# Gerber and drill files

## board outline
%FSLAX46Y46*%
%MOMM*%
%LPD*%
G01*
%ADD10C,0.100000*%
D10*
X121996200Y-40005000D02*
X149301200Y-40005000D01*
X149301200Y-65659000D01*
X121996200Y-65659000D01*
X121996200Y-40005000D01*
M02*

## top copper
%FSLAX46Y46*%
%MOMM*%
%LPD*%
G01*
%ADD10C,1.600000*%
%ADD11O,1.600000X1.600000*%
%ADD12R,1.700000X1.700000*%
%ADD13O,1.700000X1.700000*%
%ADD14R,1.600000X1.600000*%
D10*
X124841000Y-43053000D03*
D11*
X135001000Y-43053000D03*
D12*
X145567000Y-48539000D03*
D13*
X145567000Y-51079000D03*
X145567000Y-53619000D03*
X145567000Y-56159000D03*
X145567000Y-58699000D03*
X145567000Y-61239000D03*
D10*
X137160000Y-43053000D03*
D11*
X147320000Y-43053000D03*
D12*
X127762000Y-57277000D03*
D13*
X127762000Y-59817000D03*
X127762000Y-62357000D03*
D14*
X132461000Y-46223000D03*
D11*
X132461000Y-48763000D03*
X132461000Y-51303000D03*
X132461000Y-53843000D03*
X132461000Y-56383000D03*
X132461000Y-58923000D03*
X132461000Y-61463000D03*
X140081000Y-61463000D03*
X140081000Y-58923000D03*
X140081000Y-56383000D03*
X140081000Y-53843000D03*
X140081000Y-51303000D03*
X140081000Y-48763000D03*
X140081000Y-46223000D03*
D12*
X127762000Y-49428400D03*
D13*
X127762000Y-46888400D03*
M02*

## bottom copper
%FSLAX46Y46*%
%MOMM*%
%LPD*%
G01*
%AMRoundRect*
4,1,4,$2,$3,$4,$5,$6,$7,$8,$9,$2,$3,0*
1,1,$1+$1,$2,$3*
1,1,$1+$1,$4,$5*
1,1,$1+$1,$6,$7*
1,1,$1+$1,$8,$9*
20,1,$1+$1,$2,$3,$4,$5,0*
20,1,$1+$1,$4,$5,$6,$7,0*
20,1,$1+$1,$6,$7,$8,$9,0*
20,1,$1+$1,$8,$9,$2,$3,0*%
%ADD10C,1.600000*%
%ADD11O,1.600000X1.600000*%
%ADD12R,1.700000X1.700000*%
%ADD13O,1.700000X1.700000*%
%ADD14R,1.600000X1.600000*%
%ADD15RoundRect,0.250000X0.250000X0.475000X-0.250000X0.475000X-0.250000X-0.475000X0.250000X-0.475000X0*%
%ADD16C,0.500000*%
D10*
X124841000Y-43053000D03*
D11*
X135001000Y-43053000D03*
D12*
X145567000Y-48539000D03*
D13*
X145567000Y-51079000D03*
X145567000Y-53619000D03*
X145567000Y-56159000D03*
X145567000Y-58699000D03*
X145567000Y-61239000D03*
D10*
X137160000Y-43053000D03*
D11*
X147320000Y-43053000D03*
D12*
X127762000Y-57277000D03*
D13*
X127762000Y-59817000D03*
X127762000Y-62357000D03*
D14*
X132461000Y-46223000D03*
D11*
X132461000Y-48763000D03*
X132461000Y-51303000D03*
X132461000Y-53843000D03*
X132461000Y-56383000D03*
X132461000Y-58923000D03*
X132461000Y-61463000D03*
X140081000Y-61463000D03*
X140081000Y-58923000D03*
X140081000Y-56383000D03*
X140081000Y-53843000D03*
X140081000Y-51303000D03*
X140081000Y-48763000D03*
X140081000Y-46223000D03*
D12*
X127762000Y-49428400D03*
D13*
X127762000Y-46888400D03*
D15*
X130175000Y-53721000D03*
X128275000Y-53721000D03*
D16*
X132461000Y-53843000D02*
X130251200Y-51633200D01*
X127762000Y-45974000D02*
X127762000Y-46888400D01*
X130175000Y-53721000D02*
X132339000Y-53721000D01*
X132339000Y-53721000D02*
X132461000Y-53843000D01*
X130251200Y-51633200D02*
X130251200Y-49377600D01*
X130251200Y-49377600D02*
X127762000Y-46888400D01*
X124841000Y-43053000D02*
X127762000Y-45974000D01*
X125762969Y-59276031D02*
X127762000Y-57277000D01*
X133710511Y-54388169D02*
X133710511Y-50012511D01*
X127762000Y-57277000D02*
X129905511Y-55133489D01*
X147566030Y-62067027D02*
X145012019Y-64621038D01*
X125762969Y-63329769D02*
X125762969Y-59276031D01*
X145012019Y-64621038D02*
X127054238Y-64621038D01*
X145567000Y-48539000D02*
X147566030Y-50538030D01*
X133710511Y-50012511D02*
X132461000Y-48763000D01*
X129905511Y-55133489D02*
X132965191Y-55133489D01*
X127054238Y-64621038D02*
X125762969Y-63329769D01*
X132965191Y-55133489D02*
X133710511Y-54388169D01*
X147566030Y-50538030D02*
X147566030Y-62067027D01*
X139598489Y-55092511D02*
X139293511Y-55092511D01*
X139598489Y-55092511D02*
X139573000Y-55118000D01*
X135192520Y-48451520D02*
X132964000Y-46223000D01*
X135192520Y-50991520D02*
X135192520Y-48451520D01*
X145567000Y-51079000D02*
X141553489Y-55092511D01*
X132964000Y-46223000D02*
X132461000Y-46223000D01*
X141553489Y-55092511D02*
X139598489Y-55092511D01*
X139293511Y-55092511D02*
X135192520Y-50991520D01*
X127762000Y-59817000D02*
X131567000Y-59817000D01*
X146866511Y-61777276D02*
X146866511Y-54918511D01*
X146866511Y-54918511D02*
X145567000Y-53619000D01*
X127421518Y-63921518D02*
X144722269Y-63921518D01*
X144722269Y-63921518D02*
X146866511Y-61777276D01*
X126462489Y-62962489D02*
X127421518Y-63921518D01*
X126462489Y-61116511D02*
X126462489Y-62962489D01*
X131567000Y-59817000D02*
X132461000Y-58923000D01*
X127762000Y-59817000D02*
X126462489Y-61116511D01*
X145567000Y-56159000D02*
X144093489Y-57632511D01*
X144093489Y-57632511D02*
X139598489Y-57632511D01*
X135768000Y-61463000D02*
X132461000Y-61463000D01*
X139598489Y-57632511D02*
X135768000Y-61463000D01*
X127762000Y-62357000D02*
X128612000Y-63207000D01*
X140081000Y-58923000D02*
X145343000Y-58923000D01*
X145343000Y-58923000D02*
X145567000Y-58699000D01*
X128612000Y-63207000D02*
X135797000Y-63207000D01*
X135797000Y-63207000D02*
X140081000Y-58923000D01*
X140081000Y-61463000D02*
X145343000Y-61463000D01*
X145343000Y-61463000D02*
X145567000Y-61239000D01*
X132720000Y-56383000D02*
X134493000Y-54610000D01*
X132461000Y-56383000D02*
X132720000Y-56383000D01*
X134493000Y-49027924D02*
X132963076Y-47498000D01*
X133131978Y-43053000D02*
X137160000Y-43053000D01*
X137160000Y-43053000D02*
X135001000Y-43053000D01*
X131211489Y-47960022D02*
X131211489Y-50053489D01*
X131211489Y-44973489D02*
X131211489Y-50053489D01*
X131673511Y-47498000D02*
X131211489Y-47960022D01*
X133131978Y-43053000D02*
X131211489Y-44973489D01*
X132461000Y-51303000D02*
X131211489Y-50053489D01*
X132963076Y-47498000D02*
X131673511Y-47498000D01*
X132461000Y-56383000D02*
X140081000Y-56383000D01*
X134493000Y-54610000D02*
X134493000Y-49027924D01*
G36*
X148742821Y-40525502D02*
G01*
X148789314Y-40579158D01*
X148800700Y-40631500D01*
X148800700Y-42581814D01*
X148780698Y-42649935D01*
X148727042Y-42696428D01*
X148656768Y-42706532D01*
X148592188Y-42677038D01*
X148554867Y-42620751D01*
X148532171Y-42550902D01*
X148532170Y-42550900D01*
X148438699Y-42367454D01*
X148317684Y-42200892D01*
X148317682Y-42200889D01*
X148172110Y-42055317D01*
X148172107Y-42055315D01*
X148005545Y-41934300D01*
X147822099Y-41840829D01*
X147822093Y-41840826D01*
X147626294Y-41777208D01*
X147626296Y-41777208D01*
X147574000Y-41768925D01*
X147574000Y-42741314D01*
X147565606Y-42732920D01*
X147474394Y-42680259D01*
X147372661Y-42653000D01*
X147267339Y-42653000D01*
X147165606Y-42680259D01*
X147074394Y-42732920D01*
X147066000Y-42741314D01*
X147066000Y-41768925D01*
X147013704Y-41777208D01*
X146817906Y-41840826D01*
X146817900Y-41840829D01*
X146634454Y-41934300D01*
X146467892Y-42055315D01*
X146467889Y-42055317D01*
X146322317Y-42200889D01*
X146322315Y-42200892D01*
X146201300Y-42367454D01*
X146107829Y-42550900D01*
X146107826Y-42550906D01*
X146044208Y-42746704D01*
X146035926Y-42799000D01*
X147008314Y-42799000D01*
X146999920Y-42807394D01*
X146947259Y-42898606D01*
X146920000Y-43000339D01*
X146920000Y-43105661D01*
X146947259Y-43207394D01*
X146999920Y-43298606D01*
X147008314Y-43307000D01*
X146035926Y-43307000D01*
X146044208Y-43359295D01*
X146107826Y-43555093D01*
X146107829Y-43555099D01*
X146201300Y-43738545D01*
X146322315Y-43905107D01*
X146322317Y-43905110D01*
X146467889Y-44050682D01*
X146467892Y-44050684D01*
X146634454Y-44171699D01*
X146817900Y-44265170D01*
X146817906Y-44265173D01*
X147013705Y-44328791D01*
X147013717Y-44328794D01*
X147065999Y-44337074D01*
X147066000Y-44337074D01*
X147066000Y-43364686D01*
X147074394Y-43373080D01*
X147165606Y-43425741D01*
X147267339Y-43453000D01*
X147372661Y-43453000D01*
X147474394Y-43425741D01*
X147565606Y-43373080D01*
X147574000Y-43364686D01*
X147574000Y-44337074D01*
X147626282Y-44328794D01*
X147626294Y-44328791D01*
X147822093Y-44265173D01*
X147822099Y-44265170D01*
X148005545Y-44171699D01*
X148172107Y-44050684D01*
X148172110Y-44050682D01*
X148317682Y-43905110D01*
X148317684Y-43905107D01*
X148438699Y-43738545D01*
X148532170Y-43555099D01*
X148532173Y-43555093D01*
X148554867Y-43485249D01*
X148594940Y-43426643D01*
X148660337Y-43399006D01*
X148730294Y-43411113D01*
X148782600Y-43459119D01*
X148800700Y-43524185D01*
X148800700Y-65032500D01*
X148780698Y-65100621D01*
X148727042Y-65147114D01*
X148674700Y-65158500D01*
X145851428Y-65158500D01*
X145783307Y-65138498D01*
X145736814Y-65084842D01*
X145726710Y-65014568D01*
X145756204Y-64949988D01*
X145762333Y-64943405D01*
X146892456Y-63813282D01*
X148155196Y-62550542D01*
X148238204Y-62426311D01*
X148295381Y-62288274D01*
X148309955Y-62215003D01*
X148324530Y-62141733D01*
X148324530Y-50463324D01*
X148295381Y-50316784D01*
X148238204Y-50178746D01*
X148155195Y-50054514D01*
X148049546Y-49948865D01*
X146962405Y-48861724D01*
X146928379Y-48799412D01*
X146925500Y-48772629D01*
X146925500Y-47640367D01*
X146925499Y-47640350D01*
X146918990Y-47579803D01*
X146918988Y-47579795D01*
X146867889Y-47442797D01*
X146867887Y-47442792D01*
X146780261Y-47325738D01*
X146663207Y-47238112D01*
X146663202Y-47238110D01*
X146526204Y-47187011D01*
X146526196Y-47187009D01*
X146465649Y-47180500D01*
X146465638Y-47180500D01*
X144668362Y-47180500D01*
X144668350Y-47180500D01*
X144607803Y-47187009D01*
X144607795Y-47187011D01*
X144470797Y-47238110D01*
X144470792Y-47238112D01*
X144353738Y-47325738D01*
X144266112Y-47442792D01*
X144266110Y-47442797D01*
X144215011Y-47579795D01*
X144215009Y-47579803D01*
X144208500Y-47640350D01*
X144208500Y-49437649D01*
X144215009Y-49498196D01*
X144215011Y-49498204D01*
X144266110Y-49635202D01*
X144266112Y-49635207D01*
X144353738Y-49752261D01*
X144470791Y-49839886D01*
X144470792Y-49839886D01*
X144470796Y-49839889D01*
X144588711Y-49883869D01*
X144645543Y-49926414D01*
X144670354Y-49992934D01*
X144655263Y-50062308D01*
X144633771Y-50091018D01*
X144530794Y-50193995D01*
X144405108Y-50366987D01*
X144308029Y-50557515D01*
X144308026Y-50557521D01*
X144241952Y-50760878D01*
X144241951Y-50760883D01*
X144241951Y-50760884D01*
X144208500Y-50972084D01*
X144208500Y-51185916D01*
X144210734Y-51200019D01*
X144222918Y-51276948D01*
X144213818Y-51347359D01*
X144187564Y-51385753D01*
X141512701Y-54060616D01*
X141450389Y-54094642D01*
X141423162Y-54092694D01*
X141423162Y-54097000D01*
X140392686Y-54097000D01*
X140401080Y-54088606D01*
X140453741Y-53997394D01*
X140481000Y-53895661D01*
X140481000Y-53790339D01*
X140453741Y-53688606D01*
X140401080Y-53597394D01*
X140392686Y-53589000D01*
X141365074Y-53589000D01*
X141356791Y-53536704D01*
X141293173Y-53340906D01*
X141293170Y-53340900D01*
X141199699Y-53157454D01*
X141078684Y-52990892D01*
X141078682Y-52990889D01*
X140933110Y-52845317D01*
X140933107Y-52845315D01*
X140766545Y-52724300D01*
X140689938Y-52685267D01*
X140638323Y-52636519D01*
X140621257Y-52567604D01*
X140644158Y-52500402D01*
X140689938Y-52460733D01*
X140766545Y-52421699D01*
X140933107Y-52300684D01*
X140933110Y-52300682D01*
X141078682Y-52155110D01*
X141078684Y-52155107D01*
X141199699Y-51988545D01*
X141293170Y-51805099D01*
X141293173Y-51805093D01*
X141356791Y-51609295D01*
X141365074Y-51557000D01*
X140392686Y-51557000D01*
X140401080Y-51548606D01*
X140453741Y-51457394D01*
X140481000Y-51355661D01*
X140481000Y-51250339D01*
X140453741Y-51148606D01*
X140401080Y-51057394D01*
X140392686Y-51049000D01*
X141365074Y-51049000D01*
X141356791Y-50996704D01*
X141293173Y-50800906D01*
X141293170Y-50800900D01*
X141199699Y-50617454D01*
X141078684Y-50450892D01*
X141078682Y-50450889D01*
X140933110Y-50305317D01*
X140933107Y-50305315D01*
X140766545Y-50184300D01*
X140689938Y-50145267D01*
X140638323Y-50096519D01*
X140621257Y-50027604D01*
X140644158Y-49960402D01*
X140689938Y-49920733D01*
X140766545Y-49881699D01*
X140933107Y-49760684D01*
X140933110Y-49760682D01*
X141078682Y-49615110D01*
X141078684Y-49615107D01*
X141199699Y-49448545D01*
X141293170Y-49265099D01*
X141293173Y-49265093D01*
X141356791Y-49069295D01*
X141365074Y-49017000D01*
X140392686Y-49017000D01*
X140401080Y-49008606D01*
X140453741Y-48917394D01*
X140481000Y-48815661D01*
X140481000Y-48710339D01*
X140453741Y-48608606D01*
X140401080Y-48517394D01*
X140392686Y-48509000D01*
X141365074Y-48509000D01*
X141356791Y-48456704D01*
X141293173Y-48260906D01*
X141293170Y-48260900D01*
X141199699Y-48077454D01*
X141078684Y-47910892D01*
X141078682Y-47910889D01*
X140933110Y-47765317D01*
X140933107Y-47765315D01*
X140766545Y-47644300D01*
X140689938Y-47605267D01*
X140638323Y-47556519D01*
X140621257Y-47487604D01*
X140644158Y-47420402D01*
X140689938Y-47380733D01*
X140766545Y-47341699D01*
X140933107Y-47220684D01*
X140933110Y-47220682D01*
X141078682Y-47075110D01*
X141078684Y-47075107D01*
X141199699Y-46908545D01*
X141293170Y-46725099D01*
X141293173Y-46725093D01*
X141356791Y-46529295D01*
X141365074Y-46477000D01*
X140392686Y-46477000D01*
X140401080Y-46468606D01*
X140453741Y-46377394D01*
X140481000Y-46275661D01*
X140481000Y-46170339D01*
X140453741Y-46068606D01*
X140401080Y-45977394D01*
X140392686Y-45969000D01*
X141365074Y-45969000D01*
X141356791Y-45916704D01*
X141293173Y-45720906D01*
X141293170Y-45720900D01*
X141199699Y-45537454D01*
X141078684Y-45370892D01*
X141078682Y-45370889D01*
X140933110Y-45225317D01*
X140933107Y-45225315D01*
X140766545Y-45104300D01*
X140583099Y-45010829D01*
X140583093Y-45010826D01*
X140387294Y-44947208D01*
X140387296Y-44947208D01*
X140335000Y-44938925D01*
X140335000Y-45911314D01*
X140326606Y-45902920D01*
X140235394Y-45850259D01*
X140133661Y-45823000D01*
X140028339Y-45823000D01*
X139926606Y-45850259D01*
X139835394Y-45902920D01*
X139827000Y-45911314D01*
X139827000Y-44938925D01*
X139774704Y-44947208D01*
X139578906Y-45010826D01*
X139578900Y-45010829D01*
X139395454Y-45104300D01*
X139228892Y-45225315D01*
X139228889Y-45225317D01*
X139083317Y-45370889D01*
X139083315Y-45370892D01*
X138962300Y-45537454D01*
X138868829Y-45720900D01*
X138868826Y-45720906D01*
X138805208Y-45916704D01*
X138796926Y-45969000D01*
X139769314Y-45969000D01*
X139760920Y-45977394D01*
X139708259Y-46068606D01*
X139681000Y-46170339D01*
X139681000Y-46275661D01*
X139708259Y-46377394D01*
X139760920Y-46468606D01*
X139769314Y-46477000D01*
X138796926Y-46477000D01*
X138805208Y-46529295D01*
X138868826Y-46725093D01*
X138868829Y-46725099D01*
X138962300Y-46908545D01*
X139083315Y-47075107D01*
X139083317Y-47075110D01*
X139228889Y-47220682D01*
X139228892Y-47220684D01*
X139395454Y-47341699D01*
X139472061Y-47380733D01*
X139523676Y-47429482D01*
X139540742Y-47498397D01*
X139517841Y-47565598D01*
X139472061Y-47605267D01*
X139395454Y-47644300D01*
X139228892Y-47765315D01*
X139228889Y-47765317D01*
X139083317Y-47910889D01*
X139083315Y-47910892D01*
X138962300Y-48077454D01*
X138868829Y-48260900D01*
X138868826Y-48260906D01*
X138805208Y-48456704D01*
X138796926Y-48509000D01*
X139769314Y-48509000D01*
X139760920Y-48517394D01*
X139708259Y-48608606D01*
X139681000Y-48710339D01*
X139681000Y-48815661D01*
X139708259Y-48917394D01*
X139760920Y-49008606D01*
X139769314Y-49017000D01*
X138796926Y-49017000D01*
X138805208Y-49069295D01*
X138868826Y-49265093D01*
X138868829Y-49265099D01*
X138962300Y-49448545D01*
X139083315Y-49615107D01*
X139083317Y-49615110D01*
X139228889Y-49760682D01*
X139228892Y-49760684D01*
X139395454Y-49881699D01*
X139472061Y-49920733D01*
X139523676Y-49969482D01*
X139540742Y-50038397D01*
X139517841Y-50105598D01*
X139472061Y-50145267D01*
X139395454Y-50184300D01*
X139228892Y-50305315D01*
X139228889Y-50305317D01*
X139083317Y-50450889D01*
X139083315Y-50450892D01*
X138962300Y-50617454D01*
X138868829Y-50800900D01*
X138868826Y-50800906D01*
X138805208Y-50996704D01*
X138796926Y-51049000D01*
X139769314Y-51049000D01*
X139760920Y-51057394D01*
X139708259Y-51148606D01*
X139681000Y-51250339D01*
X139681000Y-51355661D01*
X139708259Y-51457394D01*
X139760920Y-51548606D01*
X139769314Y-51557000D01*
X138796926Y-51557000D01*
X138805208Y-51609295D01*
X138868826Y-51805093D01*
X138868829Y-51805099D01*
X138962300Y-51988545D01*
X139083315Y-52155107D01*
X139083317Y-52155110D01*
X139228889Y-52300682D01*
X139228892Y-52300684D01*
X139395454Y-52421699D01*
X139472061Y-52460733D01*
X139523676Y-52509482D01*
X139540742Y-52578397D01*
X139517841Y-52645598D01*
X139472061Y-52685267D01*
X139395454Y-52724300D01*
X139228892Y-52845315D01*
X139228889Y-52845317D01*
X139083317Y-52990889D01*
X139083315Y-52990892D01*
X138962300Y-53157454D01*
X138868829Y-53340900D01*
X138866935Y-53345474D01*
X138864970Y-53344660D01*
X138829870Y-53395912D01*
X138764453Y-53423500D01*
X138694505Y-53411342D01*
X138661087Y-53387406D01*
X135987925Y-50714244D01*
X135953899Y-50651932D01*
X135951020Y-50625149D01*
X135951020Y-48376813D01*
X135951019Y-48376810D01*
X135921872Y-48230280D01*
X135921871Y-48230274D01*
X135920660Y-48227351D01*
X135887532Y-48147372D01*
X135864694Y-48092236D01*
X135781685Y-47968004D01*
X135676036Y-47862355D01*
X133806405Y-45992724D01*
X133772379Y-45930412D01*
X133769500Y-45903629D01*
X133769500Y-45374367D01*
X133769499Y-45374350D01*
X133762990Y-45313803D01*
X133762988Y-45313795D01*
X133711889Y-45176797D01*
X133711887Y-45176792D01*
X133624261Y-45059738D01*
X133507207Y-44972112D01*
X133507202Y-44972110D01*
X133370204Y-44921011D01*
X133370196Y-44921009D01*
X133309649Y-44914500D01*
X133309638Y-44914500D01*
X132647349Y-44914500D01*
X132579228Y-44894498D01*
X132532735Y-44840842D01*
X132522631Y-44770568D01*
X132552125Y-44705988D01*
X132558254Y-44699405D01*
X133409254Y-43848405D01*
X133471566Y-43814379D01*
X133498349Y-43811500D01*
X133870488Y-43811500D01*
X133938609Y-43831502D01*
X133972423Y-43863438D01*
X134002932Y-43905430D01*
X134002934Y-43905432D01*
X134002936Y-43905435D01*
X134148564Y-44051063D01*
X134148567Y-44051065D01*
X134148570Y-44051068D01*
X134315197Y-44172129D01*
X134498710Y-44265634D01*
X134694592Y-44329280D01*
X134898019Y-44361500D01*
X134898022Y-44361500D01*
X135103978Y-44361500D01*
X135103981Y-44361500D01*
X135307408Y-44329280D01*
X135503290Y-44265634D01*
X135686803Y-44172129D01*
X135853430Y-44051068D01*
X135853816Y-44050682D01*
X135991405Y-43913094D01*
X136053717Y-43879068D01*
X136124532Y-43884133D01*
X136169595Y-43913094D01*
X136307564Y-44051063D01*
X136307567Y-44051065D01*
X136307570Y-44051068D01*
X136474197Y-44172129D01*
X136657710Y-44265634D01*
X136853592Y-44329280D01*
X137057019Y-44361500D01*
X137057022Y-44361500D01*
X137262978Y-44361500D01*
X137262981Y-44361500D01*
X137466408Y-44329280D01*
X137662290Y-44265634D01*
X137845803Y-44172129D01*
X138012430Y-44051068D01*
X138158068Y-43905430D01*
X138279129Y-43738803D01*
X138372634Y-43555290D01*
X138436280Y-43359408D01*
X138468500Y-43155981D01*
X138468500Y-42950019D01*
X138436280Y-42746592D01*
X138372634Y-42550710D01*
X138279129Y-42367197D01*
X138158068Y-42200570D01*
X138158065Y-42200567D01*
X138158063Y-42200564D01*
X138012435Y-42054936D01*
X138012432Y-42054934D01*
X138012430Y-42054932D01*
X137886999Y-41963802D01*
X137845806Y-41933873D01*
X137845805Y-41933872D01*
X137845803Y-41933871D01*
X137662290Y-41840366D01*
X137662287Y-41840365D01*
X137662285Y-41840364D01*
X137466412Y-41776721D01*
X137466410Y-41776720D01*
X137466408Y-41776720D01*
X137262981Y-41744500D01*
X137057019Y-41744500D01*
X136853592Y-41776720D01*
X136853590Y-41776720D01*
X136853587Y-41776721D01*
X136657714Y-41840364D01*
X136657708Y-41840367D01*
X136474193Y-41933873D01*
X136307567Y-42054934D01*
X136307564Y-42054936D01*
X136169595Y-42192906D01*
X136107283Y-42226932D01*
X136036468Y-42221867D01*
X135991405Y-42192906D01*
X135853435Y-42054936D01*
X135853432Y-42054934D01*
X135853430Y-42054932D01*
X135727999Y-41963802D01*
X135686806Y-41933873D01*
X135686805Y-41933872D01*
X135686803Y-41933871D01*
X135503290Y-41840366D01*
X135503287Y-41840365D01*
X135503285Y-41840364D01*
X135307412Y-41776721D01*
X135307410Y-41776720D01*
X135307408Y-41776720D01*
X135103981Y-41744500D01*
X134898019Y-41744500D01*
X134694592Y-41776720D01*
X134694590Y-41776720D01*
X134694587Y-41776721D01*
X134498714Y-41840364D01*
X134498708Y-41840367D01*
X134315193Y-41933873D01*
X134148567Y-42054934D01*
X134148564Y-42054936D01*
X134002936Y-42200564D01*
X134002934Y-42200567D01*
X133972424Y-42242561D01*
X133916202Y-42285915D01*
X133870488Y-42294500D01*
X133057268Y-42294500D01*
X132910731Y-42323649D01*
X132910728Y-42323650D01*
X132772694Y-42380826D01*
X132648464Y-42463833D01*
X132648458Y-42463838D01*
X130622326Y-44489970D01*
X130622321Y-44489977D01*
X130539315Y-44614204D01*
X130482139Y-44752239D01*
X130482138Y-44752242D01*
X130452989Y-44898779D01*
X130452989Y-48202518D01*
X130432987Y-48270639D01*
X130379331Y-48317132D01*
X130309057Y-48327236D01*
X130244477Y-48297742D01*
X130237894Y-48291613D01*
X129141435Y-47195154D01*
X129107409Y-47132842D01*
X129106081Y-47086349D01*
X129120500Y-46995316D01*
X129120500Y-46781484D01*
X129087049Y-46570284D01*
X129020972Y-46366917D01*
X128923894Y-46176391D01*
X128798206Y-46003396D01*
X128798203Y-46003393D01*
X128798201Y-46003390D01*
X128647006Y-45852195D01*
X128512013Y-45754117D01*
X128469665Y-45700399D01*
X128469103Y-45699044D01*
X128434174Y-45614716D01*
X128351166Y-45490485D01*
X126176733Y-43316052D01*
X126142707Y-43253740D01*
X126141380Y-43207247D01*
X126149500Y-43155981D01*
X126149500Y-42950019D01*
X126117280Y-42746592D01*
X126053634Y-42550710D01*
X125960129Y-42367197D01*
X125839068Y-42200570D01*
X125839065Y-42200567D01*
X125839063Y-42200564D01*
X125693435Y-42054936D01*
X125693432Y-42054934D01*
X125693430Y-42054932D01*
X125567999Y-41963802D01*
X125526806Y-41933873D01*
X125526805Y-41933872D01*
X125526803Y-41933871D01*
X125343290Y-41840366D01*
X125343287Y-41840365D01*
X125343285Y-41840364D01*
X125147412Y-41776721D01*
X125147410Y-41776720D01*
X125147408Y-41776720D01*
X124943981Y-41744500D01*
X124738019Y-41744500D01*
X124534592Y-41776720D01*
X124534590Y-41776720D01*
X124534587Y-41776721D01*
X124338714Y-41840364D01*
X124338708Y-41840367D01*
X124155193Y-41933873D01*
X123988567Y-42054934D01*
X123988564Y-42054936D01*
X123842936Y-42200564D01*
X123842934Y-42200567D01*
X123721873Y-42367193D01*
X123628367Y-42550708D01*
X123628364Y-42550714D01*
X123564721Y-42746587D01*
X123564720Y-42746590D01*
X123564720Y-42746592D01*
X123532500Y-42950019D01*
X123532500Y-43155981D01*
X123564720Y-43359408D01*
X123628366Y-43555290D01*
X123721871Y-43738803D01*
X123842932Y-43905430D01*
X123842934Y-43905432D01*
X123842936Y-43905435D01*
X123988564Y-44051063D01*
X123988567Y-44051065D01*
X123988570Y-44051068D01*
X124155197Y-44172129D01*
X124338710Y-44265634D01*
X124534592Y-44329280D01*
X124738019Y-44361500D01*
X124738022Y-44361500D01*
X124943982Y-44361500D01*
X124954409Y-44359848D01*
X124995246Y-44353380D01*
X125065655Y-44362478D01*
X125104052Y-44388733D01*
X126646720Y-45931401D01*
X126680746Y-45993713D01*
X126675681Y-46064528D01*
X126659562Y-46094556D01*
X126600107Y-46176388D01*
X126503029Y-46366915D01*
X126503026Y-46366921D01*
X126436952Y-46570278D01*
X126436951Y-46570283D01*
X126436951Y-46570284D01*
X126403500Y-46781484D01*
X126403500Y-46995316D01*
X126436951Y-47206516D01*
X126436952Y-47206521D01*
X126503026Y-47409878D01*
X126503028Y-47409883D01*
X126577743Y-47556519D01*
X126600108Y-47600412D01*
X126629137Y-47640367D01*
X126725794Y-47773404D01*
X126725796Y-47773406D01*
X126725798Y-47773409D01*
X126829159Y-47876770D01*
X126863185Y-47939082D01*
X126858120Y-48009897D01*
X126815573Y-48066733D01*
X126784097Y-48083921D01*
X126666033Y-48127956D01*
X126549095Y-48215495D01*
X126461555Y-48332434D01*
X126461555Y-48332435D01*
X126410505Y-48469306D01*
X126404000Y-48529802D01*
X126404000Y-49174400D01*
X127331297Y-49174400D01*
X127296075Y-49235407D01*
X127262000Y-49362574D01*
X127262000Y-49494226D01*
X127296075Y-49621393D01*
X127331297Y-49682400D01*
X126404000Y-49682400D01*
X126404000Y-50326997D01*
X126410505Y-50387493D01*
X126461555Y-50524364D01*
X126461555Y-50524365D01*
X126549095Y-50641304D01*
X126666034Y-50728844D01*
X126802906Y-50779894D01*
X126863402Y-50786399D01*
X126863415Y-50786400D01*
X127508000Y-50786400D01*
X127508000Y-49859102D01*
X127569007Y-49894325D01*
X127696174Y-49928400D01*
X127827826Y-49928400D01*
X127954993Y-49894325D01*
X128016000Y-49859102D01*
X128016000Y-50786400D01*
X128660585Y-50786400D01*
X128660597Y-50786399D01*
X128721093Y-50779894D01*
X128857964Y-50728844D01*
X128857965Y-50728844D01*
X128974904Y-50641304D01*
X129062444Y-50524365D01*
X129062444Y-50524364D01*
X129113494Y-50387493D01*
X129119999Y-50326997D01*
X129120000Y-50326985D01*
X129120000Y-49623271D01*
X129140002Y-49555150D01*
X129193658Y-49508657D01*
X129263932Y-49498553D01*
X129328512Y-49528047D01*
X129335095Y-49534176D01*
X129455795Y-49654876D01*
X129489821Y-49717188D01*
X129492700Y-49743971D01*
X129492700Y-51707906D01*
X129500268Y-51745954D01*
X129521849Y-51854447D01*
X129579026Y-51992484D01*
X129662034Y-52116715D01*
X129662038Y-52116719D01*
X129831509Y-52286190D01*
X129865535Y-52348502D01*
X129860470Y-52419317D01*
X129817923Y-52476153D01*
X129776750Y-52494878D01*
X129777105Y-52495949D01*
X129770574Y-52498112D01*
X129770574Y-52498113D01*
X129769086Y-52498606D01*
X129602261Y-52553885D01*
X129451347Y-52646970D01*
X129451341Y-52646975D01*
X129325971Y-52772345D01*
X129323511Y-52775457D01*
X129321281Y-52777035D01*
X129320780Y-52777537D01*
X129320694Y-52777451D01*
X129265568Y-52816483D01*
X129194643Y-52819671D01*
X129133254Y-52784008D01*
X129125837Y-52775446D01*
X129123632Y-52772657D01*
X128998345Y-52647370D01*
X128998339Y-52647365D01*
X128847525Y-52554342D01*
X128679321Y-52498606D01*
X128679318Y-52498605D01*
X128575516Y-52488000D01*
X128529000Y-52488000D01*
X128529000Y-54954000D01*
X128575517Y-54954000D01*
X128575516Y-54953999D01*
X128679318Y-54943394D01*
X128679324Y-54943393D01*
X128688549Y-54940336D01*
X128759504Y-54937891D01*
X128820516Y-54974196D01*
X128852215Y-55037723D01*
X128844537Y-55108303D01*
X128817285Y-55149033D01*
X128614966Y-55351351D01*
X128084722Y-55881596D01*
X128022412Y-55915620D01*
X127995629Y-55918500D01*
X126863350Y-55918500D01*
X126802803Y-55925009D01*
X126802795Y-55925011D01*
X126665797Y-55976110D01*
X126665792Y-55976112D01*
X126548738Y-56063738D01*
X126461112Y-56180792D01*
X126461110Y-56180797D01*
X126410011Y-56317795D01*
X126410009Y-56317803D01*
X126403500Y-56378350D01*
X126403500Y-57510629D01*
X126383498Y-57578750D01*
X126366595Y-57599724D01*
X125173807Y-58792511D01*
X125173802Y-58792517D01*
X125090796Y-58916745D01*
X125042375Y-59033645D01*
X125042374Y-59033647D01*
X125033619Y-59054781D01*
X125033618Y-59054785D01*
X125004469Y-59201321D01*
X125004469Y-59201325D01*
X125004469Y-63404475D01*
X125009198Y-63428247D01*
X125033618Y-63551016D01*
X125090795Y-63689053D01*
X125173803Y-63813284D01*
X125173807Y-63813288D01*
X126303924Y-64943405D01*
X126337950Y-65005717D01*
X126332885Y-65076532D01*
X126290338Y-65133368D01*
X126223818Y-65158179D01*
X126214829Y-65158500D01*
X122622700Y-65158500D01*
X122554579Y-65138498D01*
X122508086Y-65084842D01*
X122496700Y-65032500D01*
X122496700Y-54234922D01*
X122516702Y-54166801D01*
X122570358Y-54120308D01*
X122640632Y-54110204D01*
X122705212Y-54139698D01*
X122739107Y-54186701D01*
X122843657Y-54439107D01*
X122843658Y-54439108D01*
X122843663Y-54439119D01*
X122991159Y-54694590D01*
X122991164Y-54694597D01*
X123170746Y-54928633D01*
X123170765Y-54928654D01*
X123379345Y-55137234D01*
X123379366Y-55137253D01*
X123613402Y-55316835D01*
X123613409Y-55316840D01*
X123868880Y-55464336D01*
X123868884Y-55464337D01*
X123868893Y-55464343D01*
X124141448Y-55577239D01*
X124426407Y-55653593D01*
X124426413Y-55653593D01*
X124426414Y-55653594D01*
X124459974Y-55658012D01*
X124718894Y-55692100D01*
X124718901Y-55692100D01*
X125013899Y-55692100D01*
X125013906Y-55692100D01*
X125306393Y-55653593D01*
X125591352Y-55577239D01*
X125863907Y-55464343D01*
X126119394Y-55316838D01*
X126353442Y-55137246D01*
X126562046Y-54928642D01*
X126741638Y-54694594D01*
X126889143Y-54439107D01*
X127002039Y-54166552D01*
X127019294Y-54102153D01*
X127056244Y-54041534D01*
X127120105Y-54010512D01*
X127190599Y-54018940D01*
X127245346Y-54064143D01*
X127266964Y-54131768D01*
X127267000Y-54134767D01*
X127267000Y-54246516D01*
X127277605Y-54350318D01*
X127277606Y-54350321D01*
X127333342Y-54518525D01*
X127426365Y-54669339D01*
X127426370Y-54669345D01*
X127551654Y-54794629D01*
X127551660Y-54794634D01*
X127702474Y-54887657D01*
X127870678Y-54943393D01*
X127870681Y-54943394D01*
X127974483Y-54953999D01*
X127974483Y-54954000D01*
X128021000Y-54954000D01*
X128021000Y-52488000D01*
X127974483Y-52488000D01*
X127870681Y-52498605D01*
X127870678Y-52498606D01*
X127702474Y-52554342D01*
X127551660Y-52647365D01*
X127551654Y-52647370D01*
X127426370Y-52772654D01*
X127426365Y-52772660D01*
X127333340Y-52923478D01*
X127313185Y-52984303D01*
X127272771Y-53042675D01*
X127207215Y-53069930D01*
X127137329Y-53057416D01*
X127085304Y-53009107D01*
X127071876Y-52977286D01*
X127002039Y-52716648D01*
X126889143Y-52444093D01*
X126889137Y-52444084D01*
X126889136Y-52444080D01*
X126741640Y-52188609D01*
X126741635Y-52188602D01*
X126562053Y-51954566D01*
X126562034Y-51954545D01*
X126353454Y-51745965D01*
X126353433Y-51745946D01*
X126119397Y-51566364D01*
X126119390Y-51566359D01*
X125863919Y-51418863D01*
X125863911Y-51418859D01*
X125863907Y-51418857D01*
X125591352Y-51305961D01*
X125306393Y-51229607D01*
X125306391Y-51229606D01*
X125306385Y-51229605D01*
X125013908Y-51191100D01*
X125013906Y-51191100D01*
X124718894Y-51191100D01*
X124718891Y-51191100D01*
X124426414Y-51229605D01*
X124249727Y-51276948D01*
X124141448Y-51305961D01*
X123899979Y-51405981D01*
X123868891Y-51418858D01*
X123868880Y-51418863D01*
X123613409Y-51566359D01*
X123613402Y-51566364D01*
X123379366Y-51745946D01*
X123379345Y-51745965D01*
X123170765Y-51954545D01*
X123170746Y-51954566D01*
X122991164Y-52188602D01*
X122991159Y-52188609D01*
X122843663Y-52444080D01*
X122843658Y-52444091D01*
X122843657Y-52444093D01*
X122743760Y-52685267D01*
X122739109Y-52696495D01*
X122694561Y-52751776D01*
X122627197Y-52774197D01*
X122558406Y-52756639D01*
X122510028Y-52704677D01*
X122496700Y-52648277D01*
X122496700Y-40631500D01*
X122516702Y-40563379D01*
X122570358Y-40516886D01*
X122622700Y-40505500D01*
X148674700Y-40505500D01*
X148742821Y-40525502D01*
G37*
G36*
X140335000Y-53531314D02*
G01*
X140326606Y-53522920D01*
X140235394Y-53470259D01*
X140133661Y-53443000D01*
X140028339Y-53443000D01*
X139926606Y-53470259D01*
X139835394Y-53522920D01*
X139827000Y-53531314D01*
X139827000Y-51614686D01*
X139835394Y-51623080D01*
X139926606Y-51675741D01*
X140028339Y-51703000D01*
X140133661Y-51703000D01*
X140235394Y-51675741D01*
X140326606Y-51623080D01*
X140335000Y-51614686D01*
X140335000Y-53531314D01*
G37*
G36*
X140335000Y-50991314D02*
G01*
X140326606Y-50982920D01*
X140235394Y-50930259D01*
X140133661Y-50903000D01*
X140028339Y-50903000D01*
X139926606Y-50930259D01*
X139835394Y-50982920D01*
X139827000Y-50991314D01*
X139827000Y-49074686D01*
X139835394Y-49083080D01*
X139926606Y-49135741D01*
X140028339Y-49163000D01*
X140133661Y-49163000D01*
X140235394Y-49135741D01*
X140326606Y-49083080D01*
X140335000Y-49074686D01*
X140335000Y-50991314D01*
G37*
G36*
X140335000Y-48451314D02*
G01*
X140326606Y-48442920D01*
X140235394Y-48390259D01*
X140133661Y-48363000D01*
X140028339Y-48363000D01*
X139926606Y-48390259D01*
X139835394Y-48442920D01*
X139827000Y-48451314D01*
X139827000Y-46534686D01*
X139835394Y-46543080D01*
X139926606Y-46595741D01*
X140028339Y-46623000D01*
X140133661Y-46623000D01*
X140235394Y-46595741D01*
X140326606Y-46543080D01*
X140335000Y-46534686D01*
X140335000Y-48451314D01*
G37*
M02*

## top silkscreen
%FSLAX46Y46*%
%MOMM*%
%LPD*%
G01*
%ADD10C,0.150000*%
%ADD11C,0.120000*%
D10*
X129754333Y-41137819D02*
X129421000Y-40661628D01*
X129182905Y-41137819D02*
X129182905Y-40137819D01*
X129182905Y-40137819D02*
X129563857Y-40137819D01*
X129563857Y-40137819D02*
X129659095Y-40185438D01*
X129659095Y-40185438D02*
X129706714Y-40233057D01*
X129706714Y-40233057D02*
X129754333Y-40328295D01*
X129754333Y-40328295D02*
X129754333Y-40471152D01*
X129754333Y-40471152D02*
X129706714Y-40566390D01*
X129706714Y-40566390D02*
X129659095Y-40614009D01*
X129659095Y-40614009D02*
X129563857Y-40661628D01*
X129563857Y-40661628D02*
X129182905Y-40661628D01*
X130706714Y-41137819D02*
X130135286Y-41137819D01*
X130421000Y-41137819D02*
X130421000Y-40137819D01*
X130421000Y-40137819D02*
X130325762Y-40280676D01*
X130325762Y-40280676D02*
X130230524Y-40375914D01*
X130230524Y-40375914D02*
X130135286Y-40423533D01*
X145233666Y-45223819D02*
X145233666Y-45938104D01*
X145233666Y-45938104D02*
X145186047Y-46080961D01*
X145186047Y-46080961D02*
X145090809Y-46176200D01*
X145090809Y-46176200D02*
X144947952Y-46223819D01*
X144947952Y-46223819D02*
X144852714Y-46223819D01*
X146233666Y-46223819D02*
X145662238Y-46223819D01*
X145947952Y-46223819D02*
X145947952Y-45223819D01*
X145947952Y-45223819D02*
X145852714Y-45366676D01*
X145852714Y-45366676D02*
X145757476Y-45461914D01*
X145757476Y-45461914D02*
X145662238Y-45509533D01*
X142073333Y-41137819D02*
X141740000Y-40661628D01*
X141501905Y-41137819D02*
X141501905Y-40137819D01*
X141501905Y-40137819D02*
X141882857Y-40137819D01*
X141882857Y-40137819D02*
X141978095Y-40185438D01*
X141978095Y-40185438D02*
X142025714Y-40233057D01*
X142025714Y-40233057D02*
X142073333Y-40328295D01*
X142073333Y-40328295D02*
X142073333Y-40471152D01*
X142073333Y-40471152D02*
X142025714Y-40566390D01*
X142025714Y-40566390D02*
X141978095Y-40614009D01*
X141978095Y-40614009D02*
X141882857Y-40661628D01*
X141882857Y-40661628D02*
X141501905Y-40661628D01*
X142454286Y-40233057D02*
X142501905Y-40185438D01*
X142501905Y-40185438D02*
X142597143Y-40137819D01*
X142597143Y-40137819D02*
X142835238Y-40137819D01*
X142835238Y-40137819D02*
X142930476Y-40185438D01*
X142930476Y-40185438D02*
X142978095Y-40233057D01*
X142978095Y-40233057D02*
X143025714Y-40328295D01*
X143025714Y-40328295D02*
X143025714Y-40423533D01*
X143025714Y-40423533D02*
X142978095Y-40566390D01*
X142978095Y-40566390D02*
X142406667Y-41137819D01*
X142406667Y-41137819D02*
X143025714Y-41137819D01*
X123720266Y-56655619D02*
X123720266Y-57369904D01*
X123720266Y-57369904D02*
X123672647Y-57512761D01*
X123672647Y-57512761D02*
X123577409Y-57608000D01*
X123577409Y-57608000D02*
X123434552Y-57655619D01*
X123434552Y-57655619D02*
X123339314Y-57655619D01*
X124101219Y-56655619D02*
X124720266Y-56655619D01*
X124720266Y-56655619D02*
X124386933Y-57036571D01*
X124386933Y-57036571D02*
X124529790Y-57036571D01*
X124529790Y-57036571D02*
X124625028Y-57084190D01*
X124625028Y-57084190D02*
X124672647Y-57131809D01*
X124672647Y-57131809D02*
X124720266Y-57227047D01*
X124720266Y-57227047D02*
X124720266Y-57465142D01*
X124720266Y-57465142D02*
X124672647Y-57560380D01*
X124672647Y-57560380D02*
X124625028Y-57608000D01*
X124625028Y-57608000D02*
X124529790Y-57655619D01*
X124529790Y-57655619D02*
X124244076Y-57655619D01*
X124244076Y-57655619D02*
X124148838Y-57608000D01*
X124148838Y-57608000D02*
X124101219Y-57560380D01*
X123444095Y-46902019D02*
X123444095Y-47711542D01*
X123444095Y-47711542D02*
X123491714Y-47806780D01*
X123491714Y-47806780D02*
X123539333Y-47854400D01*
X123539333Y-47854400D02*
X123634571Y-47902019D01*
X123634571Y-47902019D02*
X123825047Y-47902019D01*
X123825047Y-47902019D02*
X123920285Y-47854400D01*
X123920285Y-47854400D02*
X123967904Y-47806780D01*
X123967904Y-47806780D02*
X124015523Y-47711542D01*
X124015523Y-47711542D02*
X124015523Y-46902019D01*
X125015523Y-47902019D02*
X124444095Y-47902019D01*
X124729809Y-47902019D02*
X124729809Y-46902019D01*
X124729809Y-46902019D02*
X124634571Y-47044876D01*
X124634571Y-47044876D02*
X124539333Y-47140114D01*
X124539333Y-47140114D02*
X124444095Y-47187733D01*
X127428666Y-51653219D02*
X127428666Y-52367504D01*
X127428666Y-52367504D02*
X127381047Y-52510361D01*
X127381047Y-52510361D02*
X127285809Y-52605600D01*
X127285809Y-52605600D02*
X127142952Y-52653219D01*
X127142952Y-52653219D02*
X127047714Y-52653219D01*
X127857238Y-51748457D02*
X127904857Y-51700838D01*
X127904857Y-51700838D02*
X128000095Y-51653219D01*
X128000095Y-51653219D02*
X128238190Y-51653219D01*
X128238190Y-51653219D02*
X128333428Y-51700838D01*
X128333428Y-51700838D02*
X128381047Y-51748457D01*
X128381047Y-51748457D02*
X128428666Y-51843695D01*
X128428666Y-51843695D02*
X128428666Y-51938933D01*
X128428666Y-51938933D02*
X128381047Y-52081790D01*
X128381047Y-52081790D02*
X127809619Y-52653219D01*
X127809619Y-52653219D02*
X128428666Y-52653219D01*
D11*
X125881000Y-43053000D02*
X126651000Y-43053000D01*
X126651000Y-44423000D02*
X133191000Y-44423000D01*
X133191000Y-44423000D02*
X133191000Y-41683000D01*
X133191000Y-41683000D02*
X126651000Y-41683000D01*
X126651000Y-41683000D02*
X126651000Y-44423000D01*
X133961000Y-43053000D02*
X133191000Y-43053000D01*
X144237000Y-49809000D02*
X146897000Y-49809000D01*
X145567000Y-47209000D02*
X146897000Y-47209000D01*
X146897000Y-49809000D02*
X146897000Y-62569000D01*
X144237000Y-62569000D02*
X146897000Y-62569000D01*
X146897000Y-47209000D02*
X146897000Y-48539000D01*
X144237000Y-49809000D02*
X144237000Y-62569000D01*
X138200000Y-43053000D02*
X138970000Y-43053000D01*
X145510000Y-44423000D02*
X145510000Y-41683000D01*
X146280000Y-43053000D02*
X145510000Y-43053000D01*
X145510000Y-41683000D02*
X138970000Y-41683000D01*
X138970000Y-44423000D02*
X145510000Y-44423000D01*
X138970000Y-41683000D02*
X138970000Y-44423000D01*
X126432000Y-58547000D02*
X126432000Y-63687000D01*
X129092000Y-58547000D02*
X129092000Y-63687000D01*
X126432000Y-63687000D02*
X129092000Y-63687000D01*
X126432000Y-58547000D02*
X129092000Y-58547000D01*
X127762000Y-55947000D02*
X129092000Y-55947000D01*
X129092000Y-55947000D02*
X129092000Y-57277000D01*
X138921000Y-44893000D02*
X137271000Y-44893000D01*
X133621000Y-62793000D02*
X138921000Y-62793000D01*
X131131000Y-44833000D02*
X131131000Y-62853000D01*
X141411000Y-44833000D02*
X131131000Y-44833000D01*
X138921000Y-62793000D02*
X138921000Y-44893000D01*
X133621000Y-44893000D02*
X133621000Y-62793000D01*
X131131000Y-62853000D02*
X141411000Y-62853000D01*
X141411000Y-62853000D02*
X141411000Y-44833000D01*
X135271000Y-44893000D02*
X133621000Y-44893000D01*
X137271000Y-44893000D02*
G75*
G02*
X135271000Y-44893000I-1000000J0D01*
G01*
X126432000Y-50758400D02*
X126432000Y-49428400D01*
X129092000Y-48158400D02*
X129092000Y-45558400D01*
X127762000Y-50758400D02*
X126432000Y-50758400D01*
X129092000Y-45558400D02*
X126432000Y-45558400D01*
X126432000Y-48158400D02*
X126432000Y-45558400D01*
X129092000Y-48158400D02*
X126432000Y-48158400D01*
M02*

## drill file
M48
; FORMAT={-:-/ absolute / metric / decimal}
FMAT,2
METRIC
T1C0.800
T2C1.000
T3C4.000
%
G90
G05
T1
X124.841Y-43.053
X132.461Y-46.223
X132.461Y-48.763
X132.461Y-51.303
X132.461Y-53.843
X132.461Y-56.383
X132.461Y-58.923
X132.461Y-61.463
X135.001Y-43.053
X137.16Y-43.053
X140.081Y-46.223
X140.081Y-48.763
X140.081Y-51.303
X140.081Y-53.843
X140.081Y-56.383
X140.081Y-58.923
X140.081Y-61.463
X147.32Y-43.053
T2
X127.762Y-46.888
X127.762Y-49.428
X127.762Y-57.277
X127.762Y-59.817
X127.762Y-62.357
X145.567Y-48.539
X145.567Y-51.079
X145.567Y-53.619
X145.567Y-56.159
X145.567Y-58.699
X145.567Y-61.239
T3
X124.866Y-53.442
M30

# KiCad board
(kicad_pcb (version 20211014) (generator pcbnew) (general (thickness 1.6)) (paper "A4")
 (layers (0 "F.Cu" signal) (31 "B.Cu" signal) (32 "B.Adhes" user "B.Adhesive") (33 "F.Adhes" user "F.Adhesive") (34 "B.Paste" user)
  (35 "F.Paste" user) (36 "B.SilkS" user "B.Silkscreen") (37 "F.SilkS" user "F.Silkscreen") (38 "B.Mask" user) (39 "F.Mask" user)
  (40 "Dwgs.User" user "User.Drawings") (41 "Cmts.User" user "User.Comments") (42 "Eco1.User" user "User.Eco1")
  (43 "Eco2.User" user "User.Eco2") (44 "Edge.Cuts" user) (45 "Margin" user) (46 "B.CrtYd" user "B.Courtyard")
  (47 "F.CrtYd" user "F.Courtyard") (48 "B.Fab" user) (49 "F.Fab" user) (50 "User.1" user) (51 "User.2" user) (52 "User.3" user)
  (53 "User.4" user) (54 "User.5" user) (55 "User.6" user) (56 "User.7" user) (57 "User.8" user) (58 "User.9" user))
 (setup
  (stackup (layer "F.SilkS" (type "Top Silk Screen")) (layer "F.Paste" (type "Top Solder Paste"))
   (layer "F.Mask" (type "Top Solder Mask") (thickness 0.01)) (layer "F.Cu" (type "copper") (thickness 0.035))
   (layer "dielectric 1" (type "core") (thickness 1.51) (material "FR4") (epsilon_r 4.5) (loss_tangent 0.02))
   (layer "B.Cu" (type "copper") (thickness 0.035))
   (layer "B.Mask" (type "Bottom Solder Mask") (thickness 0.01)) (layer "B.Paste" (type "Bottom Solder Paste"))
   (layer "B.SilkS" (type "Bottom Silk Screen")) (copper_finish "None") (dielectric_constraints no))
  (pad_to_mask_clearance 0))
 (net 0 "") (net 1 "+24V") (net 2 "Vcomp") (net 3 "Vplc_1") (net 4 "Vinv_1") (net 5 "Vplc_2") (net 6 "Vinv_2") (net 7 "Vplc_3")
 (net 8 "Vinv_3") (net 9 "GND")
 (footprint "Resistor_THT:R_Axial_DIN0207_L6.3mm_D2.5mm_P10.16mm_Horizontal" (layer "F.Cu") (at 124.841 43.053)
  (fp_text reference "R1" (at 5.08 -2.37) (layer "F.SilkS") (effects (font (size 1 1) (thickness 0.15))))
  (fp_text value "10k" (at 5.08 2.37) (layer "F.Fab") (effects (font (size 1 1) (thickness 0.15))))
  (fp_line (start 1.04 0) (end 1.81 0) (layer "F.SilkS") (width 0.12))
  (fp_line (start 1.81 1.37) (end 8.35 1.37) (layer "F.SilkS") (width 0.12))
  (fp_line (start 8.35 1.37) (end 8.35 -1.37) (layer "F.SilkS") (width 0.12))
  (fp_line (start 8.35 -1.37) (end 1.81 -1.37) (layer "F.SilkS") (width 0.12))
  (fp_line (start 1.81 -1.37) (end 1.81 1.37) (layer "F.SilkS") (width 0.12))
  (fp_line (start 9.12 0) (end 8.35 0) (layer "F.SilkS") (width 0.12))
  (pad "1" thru_hole circle (at 0 0) (size 1.6 1.6) (drill 0.8) (layers *.Cu *.Mask) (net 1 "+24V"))
  (pad "2" thru_hole oval (at 10.16 0) (size 1.6 1.6) (drill 0.8) (layers *.Cu *.Mask) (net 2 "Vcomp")))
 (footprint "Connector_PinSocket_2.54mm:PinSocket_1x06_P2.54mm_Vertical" (layer "F.Cu") (at 145.567 48.539)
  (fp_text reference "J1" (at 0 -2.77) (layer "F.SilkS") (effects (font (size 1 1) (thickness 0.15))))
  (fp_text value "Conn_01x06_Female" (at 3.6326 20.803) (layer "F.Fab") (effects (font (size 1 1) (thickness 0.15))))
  (fp_line (start -1.33 1.27) (end 1.33 1.27) (layer "F.SilkS") (width 0.12))
  (fp_line (start 0 -1.33) (end 1.33 -1.33) (layer "F.SilkS") (width 0.12))
  (fp_line (start 1.33 1.27) (end 1.33 14.03) (layer "F.SilkS") (width 0.12))
  (fp_line (start -1.33 14.03) (end 1.33 14.03) (layer "F.SilkS") (width 0.12))
  (fp_line (start 1.33 -1.33) (end 1.33 0) (layer "F.SilkS") (width 0.12))
  (fp_line (start -1.33 1.27) (end -1.33 14.03) (layer "F.SilkS") (width 0.12))
  (pad "1" thru_hole rect (at 0 0) (size 1.7 1.7) (drill 1) (layers *.Cu *.Mask) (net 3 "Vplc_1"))
  (pad "2" thru_hole oval (at 0 2.54) (size 1.7 1.7) (drill 1) (layers *.Cu *.Mask) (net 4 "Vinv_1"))
  (pad "3" thru_hole oval (at 0 5.08) (size 1.7 1.7) (drill 1) (layers *.Cu *.Mask) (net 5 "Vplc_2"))
  (pad "4" thru_hole oval (at 0 7.62) (size 1.7 1.7) (drill 1) (layers *.Cu *.Mask) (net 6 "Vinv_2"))
  (pad "5" thru_hole oval (at 0 10.16) (size 1.7 1.7) (drill 1) (layers *.Cu *.Mask) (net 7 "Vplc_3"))
  (pad "6" thru_hole oval (at 0 12.7) (size 1.7 1.7) (drill 1) (layers *.Cu *.Mask) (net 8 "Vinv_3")))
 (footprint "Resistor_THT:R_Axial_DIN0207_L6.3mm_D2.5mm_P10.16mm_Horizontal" (layer "F.Cu") (at 137.16 43.053)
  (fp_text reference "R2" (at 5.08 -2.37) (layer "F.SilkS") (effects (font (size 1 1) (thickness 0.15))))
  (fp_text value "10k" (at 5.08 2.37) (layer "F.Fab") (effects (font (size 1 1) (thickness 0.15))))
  (fp_line (start 1.04 0) (end 1.81 0) (layer "F.SilkS") (width 0.12))
  (fp_line (start 8.35 1.37) (end 8.35 -1.37) (layer "F.SilkS") (width 0.12))
  (fp_line (start 9.12 0) (end 8.35 0) (layer "F.SilkS") (width 0.12))
  (fp_line (start 8.35 -1.37) (end 1.81 -1.37) (layer "F.SilkS") (width 0.12))
  (fp_line (start 1.81 1.37) (end 8.35 1.37) (layer "F.SilkS") (width 0.12))
  (fp_line (start 1.81 -1.37) (end 1.81 1.37) (layer "F.SilkS") (width 0.12))
  (pad "1" thru_hole circle (at 0 0) (size 1.6 1.6) (drill 0.8) (layers *.Cu *.Mask) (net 2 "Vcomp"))
  (pad "2" thru_hole oval (at 10.16 0) (size 1.6 1.6) (drill 0.8) (layers *.Cu *.Mask) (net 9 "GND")))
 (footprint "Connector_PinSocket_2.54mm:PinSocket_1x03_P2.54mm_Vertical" (layer "F.Cu") (at 127.762 57.277)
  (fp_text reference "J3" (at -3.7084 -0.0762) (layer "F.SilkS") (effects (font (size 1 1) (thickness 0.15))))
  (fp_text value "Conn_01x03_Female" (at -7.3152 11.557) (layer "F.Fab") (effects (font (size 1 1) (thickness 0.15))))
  (fp_line (start -1.33 1.27) (end -1.33 6.41) (layer "F.SilkS") (width 0.12))
  (fp_line (start 1.33 1.27) (end 1.33 6.41) (layer "F.SilkS") (width 0.12))
  (fp_line (start -1.33 6.41) (end 1.33 6.41) (layer "F.SilkS") (width 0.12))
  (fp_line (start -1.33 1.27) (end 1.33 1.27) (layer "F.SilkS") (width 0.12))
  (fp_line (start 0 -1.33) (end 1.33 -1.33) (layer "F.SilkS") (width 0.12))
  (fp_line (start 1.33 -1.33) (end 1.33 0) (layer "F.SilkS") (width 0.12))
  (pad "1" thru_hole rect (at 0 0) (size 1.7 1.7) (drill 1) (layers *.Cu *.Mask) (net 3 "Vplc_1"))
  (pad "2" thru_hole oval (at 0 2.54) (size 1.7 1.7) (drill 1) (layers *.Cu *.Mask) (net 5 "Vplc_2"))
  (pad "3" thru_hole oval (at 0 5.08) (size 1.7 1.7) (drill 1) (layers *.Cu *.Mask) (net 7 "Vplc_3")))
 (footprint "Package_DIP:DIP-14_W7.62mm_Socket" (layer "F.Cu") (at 132.461 46.223)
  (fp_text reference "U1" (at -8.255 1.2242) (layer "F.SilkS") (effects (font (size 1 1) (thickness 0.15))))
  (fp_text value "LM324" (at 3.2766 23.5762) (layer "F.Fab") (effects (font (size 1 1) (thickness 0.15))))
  (fp_line (start 6.46 -1.33) (end 4.81 -1.33) (layer "F.SilkS") (width 0.12))
  (fp_line (start 1.16 16.57) (end 6.46 16.57) (layer "F.SilkS") (width 0.12))
  (fp_line (start -1.33 -1.39) (end -1.33 16.63) (layer "F.SilkS") (width 0.12))
  (fp_line (start 8.95 -1.39) (end -1.33 -1.39) (layer "F.SilkS") (width 0.12))
  (fp_line (start 6.46 16.57) (end 6.46 -1.33) (layer "F.SilkS") (width 0.12))
  (fp_line (start 1.16 -1.33) (end 1.16 16.57) (layer "F.SilkS") (width 0.12))
  (fp_line (start -1.33 16.63) (end 8.95 16.63) (layer "F.SilkS") (width 0.12))
  (fp_line (start 8.95 16.63) (end 8.95 -1.39) (layer "F.SilkS") (width 0.12))
  (fp_line (start 2.81 -1.33) (end 1.16 -1.33) (layer "F.SilkS") (width 0.12))
  (fp_arc (start 4.81 -1.33) (mid 3.81 -0.33) (end 2.81 -1.33) (layer "F.SilkS") (width 0.12))
  (pad "1" thru_hole rect (at 0 0) (size 1.6 1.6) (drill 0.8) (layers *.Cu *.Mask) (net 4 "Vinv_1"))
  (pad "2" thru_hole oval (at 0 2.54) (size 1.6 1.6) (drill 0.8) (layers *.Cu *.Mask) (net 3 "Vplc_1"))
  (pad "3" thru_hole oval (at 0 5.08) (size 1.6 1.6) (drill 0.8) (layers *.Cu *.Mask) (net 2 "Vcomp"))
  (pad "4" thru_hole oval (at 0 7.62) (size 1.6 1.6) (drill 0.8) (layers *.Cu *.Mask) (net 1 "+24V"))
  (pad "5" thru_hole oval (at 0 10.16) (size 1.6 1.6) (drill 0.8) (layers *.Cu *.Mask) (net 2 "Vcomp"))
  (pad "6" thru_hole oval (at 0 12.7) (size 1.6 1.6) (drill 0.8) (layers *.Cu *.Mask) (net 5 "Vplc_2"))
  (pad "7" thru_hole oval (at 0 15.24) (size 1.6 1.6) (drill 0.8) (layers *.Cu *.Mask) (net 6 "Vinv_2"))
  (pad "8" thru_hole oval (at 7.62 15.24) (size 1.6 1.6) (drill 0.8) (layers *.Cu *.Mask) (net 8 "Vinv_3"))
  (pad "9" thru_hole oval (at 7.62 12.7) (size 1.6 1.6) (drill 0.8) (layers *.Cu *.Mask) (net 7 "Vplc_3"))
  (pad "10" thru_hole oval (at 7.62 10.16) (size 1.6 1.6) (drill 0.8) (layers *.Cu *.Mask) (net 2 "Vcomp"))
  (pad "11" thru_hole oval (at 7.62 7.62) (size 1.6 1.6) (drill 0.8) (layers *.Cu *.Mask) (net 9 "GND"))
  (pad "12" thru_hole oval (at 7.62 5.08) (size 1.6 1.6) (drill 0.8) (layers *.Cu *.Mask) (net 9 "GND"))
  (pad "13" thru_hole oval (at 7.62 2.54) (size 1.6 1.6) (drill 0.8) (layers *.Cu *.Mask) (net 9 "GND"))
  (pad "14" thru_hole oval (at 7.62 0) (size 1.6 1.6) (drill 0.8) (layers *.Cu *.Mask) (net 9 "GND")))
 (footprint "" (layer "F.Cu") (at 124.8664 53.4416)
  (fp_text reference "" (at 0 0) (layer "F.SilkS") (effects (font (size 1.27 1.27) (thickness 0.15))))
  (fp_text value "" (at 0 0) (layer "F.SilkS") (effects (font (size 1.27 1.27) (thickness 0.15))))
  (pad "" np_thru_hole circle (at 0 0) (size 4 4) (drill 4) (layers *.Cu *.Mask)))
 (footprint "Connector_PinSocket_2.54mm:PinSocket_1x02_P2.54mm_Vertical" (layer "F.Cu") (at 127.762 49.4284 180)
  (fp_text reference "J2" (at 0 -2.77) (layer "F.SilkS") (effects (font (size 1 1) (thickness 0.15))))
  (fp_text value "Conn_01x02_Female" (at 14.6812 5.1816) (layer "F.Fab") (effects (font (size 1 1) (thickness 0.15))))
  (fp_line (start 1.33 -1.33) (end 1.33 0) (layer "F.SilkS") (width 0.12))
  (fp_line (start -1.33 1.27) (end -1.33 3.87) (layer "F.SilkS") (width 0.12))
  (fp_line (start 0 -1.33) (end 1.33 -1.33) (layer "F.SilkS") (width 0.12))
  (fp_line (start -1.33 3.87) (end 1.33 3.87) (layer "F.SilkS") (width 0.12))
  (fp_line (start 1.33 1.27) (end 1.33 3.87) (layer "F.SilkS") (width 0.12))
  (fp_line (start -1.33 1.27) (end 1.33 1.27) (layer "F.SilkS") (width 0.12))
  (pad "1" thru_hole rect (at 0 0 180) (size 1.7 1.7) (drill 1) (layers *.Cu *.Mask) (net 9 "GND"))
  (pad "2" thru_hole oval (at 0 2.54 180) (size 1.7 1.7) (drill 1) (layers *.Cu *.Mask) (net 1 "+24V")))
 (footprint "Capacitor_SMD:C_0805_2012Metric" (layer "B.Cu") (at 129.225 53.721 180)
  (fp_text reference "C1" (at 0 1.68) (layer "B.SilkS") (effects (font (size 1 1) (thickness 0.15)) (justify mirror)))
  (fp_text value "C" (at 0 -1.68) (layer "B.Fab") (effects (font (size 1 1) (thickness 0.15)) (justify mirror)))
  (pad "1" smd roundrect (at -0.95 0 180) (size 1 1.45) (layers "B.Cu" "B.Paste" "B.Mask") (roundrect_rratio 0.25) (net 1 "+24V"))
  (pad "2" smd roundrect (at 0.95 0 180) (size 1 1.45) (layers "B.Cu" "B.Paste" "B.Mask") (roundrect_rratio 0.25) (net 9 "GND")))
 (gr_rect (start 121.9962 40.005) (end 149.3012 65.659) (layer "Edge.Cuts") (width 0.1) (fill none))
 (segment (start 132.461 53.843) (end 130.2512 51.6332) (width 0.5) (layer "B.Cu") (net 1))
 (segment (start 127.762 45.974) (end 127.762 46.8884) (width 0.5) (layer "B.Cu") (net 1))
 (segment (start 130.175 53.721) (end 132.339 53.721) (width 0.5) (layer "B.Cu") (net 1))
 (segment (start 132.339 53.721) (end 132.461 53.843) (width 0.5) (layer "B.Cu") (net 1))
 (segment (start 130.2512 51.6332) (end 130.2512 49.3776) (width 0.5) (layer "B.Cu") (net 1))
 (segment (start 130.2512 49.3776) (end 127.762 46.8884) (width 0.5) (layer "B.Cu") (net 1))
 (segment (start 124.841 43.053) (end 127.762 45.974) (width 0.5) (layer "B.Cu") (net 1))
 (segment (start 125.762969 59.276031) (end 127.762 57.277) (width 0.5) (layer "B.Cu") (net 3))
 (segment (start 133.710511 54.388169) (end 133.710511 50.012511) (width 0.5) (layer "B.Cu") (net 3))
 (segment (start 127.762 57.277) (end 129.905511 55.133489) (width 0.5) (layer "B.Cu") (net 3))
 (segment (start 147.56603 62.067027) (end 145.012019 64.621038) (width 0.5) (layer "B.Cu") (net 3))
 (segment (start 125.762969 63.329769) (end 125.762969 59.276031) (width 0.5) (layer "B.Cu") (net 3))
 (segment (start 145.012019 64.621038) (end 127.054238 64.621038) (width 0.5) (layer "B.Cu") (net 3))
 (segment (start 145.567 48.539) (end 147.56603 50.53803) (width 0.5) (layer "B.Cu") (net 3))
 (segment (start 133.710511 50.012511) (end 132.461 48.763) (width 0.5) (layer "B.Cu") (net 3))
 (segment (start 129.905511 55.133489) (end 132.965191 55.133489) (width 0.5) (layer "B.Cu") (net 3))
 (segment (start 127.054238 64.621038) (end 125.762969 63.329769) (width 0.5) (layer "B.Cu") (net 3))
 (segment (start 132.965191 55.133489) (end 133.710511 54.388169) (width 0.5) (layer "B.Cu") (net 3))
 (segment (start 147.56603 50.53803) (end 147.56603 62.067027) (width 0.5) (layer "B.Cu") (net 3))
 (segment (start 139.598489 55.092511) (end 139.293511 55.092511) (width 0.5) (layer "B.Cu") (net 4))
 (segment (start 139.598489 55.092511) (end 139.573 55.118) (width 0.5) (layer "B.Cu") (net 4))
 (segment (start 135.19252 48.45152) (end 132.964 46.223) (width 0.5) (layer "B.Cu") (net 4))
 (segment (start 135.19252 50.99152) (end 135.19252 48.45152) (width 0.5) (layer "B.Cu") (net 4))
 (segment (start 145.567 51.079) (end 141.553489 55.092511) (width 0.5) (layer "B.Cu") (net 4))
 (segment (start 132.964 46.223) (end 132.461 46.223) (width 0.5) (layer "B.Cu") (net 4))
 (segment (start 141.553489 55.092511) (end 139.598489 55.092511) (width 0.5) (layer "B.Cu") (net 4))
 (segment (start 139.293511 55.092511) (end 135.19252 50.99152) (width 0.5) (layer "B.Cu") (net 4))
 (segment (start 127.762 59.817) (end 131.567 59.817) (width 0.5) (layer "B.Cu") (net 5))
 (segment (start 146.866511 61.777276) (end 146.866511 54.918511) (width 0.5) (layer "B.Cu") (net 5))
 (segment (start 146.866511 54.918511) (end 145.567 53.619) (width 0.5) (layer "B.Cu") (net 5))
 (segment (start 127.421518 63.921518) (end 144.722269 63.921518) (width 0.5) (layer "B.Cu") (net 5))
 (segment (start 144.722269 63.921518) (end 146.866511 61.777276) (width 0.5) (layer "B.Cu") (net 5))
 (segment (start 126.462489 62.962489) (end 127.421518 63.921518) (width 0.5) (layer "B.Cu") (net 5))
 (segment (start 126.462489 61.116511) (end 126.462489 62.962489) (width 0.5) (layer "B.Cu") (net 5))
 (segment (start 131.567 59.817) (end 132.461 58.923) (width 0.5) (layer "B.Cu") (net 5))
 (segment (start 127.762 59.817) (end 126.462489 61.116511) (width 0.5) (layer "B.Cu") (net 5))
 (segment (start 145.567 56.159) (end 144.093489 57.632511) (width 0.5) (layer "B.Cu") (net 6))
 (segment (start 144.093489 57.632511) (end 139.598489 57.632511) (width 0.5) (layer "B.Cu") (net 6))
 (segment (start 135.768 61.463) (end 132.461 61.463) (width 0.5) (layer "B.Cu") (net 6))
 (segment (start 139.598489 57.632511) (end 135.768 61.463) (width 0.5) (layer "B.Cu") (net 6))
 (segment (start 127.762 62.357) (end 128.612 63.207) (width 0.5) (layer "B.Cu") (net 7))
 (segment (start 140.081 58.923) (end 145.343 58.923) (width 0.5) (layer "B.Cu") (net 7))
 (segment (start 145.343 58.923) (end 145.567 58.699) (width 0.5) (layer "B.Cu") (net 7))
 (segment (start 128.612 63.207) (end 135.797 63.207) (width 0.5) (layer "B.Cu") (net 7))
 (segment (start 135.797 63.207) (end 140.081 58.923) (width 0.5) (layer "B.Cu") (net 7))
 (segment (start 140.081 61.463) (end 145.343 61.463) (width 0.5) (layer "B.Cu") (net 8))
 (segment (start 145.343 61.463) (end 145.567 61.239) (width 0.5) (layer "B.Cu") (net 8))
 (segment (start 132.72 56.383) (end 134.493 54.61) (width 0.5) (layer "B.Cu") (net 2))
 (segment (start 132.461 56.383) (end 132.72 56.383) (width 0.5) (layer "B.Cu") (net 2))
 (segment (start 134.493 49.027924) (end 132.963076 47.498) (width 0.5) (layer "B.Cu") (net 2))
 (segment (start 133.131978 43.053) (end 137.16 43.053) (width 0.5) (layer "B.Cu") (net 2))
 (segment (start 137.16 43.053) (end 135.001 43.053) (width 0.5) (layer "B.Cu") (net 2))
 (segment (start 131.211489 47.960022) (end 131.211489 50.053489) (width 0.5) (layer "B.Cu") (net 2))
 (segment (start 131.211489 44.973489) (end 131.211489 50.053489) (width 0.5) (layer "B.Cu") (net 2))
 (segment (start 131.673511 47.498) (end 131.211489 47.960022) (width 0.5) (layer "B.Cu") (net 2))
 (segment (start 133.131978 43.053) (end 131.211489 44.973489) (width 0.5) (layer "B.Cu") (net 2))
 (segment (start 132.461 51.303) (end 131.211489 50.053489) (width 0.5) (layer "B.Cu") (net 2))
 (segment (start 132.963076 47.498) (end 131.673511 47.498) (width 0.5) (layer "B.Cu") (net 2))
 (segment (start 132.461 56.383) (end 140.081 56.383) (width 0.5) (layer "B.Cu") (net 2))
 (segment (start 134.493 54.61) (end 134.493 49.027924) (width 0.5) (layer "B.Cu") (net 2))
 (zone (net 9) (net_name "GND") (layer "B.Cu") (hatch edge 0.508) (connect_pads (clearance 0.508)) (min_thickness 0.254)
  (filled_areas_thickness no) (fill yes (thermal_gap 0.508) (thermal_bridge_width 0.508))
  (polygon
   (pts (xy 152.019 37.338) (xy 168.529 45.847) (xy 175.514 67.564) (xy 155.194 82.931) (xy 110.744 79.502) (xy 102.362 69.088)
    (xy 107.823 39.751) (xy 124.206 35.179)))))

